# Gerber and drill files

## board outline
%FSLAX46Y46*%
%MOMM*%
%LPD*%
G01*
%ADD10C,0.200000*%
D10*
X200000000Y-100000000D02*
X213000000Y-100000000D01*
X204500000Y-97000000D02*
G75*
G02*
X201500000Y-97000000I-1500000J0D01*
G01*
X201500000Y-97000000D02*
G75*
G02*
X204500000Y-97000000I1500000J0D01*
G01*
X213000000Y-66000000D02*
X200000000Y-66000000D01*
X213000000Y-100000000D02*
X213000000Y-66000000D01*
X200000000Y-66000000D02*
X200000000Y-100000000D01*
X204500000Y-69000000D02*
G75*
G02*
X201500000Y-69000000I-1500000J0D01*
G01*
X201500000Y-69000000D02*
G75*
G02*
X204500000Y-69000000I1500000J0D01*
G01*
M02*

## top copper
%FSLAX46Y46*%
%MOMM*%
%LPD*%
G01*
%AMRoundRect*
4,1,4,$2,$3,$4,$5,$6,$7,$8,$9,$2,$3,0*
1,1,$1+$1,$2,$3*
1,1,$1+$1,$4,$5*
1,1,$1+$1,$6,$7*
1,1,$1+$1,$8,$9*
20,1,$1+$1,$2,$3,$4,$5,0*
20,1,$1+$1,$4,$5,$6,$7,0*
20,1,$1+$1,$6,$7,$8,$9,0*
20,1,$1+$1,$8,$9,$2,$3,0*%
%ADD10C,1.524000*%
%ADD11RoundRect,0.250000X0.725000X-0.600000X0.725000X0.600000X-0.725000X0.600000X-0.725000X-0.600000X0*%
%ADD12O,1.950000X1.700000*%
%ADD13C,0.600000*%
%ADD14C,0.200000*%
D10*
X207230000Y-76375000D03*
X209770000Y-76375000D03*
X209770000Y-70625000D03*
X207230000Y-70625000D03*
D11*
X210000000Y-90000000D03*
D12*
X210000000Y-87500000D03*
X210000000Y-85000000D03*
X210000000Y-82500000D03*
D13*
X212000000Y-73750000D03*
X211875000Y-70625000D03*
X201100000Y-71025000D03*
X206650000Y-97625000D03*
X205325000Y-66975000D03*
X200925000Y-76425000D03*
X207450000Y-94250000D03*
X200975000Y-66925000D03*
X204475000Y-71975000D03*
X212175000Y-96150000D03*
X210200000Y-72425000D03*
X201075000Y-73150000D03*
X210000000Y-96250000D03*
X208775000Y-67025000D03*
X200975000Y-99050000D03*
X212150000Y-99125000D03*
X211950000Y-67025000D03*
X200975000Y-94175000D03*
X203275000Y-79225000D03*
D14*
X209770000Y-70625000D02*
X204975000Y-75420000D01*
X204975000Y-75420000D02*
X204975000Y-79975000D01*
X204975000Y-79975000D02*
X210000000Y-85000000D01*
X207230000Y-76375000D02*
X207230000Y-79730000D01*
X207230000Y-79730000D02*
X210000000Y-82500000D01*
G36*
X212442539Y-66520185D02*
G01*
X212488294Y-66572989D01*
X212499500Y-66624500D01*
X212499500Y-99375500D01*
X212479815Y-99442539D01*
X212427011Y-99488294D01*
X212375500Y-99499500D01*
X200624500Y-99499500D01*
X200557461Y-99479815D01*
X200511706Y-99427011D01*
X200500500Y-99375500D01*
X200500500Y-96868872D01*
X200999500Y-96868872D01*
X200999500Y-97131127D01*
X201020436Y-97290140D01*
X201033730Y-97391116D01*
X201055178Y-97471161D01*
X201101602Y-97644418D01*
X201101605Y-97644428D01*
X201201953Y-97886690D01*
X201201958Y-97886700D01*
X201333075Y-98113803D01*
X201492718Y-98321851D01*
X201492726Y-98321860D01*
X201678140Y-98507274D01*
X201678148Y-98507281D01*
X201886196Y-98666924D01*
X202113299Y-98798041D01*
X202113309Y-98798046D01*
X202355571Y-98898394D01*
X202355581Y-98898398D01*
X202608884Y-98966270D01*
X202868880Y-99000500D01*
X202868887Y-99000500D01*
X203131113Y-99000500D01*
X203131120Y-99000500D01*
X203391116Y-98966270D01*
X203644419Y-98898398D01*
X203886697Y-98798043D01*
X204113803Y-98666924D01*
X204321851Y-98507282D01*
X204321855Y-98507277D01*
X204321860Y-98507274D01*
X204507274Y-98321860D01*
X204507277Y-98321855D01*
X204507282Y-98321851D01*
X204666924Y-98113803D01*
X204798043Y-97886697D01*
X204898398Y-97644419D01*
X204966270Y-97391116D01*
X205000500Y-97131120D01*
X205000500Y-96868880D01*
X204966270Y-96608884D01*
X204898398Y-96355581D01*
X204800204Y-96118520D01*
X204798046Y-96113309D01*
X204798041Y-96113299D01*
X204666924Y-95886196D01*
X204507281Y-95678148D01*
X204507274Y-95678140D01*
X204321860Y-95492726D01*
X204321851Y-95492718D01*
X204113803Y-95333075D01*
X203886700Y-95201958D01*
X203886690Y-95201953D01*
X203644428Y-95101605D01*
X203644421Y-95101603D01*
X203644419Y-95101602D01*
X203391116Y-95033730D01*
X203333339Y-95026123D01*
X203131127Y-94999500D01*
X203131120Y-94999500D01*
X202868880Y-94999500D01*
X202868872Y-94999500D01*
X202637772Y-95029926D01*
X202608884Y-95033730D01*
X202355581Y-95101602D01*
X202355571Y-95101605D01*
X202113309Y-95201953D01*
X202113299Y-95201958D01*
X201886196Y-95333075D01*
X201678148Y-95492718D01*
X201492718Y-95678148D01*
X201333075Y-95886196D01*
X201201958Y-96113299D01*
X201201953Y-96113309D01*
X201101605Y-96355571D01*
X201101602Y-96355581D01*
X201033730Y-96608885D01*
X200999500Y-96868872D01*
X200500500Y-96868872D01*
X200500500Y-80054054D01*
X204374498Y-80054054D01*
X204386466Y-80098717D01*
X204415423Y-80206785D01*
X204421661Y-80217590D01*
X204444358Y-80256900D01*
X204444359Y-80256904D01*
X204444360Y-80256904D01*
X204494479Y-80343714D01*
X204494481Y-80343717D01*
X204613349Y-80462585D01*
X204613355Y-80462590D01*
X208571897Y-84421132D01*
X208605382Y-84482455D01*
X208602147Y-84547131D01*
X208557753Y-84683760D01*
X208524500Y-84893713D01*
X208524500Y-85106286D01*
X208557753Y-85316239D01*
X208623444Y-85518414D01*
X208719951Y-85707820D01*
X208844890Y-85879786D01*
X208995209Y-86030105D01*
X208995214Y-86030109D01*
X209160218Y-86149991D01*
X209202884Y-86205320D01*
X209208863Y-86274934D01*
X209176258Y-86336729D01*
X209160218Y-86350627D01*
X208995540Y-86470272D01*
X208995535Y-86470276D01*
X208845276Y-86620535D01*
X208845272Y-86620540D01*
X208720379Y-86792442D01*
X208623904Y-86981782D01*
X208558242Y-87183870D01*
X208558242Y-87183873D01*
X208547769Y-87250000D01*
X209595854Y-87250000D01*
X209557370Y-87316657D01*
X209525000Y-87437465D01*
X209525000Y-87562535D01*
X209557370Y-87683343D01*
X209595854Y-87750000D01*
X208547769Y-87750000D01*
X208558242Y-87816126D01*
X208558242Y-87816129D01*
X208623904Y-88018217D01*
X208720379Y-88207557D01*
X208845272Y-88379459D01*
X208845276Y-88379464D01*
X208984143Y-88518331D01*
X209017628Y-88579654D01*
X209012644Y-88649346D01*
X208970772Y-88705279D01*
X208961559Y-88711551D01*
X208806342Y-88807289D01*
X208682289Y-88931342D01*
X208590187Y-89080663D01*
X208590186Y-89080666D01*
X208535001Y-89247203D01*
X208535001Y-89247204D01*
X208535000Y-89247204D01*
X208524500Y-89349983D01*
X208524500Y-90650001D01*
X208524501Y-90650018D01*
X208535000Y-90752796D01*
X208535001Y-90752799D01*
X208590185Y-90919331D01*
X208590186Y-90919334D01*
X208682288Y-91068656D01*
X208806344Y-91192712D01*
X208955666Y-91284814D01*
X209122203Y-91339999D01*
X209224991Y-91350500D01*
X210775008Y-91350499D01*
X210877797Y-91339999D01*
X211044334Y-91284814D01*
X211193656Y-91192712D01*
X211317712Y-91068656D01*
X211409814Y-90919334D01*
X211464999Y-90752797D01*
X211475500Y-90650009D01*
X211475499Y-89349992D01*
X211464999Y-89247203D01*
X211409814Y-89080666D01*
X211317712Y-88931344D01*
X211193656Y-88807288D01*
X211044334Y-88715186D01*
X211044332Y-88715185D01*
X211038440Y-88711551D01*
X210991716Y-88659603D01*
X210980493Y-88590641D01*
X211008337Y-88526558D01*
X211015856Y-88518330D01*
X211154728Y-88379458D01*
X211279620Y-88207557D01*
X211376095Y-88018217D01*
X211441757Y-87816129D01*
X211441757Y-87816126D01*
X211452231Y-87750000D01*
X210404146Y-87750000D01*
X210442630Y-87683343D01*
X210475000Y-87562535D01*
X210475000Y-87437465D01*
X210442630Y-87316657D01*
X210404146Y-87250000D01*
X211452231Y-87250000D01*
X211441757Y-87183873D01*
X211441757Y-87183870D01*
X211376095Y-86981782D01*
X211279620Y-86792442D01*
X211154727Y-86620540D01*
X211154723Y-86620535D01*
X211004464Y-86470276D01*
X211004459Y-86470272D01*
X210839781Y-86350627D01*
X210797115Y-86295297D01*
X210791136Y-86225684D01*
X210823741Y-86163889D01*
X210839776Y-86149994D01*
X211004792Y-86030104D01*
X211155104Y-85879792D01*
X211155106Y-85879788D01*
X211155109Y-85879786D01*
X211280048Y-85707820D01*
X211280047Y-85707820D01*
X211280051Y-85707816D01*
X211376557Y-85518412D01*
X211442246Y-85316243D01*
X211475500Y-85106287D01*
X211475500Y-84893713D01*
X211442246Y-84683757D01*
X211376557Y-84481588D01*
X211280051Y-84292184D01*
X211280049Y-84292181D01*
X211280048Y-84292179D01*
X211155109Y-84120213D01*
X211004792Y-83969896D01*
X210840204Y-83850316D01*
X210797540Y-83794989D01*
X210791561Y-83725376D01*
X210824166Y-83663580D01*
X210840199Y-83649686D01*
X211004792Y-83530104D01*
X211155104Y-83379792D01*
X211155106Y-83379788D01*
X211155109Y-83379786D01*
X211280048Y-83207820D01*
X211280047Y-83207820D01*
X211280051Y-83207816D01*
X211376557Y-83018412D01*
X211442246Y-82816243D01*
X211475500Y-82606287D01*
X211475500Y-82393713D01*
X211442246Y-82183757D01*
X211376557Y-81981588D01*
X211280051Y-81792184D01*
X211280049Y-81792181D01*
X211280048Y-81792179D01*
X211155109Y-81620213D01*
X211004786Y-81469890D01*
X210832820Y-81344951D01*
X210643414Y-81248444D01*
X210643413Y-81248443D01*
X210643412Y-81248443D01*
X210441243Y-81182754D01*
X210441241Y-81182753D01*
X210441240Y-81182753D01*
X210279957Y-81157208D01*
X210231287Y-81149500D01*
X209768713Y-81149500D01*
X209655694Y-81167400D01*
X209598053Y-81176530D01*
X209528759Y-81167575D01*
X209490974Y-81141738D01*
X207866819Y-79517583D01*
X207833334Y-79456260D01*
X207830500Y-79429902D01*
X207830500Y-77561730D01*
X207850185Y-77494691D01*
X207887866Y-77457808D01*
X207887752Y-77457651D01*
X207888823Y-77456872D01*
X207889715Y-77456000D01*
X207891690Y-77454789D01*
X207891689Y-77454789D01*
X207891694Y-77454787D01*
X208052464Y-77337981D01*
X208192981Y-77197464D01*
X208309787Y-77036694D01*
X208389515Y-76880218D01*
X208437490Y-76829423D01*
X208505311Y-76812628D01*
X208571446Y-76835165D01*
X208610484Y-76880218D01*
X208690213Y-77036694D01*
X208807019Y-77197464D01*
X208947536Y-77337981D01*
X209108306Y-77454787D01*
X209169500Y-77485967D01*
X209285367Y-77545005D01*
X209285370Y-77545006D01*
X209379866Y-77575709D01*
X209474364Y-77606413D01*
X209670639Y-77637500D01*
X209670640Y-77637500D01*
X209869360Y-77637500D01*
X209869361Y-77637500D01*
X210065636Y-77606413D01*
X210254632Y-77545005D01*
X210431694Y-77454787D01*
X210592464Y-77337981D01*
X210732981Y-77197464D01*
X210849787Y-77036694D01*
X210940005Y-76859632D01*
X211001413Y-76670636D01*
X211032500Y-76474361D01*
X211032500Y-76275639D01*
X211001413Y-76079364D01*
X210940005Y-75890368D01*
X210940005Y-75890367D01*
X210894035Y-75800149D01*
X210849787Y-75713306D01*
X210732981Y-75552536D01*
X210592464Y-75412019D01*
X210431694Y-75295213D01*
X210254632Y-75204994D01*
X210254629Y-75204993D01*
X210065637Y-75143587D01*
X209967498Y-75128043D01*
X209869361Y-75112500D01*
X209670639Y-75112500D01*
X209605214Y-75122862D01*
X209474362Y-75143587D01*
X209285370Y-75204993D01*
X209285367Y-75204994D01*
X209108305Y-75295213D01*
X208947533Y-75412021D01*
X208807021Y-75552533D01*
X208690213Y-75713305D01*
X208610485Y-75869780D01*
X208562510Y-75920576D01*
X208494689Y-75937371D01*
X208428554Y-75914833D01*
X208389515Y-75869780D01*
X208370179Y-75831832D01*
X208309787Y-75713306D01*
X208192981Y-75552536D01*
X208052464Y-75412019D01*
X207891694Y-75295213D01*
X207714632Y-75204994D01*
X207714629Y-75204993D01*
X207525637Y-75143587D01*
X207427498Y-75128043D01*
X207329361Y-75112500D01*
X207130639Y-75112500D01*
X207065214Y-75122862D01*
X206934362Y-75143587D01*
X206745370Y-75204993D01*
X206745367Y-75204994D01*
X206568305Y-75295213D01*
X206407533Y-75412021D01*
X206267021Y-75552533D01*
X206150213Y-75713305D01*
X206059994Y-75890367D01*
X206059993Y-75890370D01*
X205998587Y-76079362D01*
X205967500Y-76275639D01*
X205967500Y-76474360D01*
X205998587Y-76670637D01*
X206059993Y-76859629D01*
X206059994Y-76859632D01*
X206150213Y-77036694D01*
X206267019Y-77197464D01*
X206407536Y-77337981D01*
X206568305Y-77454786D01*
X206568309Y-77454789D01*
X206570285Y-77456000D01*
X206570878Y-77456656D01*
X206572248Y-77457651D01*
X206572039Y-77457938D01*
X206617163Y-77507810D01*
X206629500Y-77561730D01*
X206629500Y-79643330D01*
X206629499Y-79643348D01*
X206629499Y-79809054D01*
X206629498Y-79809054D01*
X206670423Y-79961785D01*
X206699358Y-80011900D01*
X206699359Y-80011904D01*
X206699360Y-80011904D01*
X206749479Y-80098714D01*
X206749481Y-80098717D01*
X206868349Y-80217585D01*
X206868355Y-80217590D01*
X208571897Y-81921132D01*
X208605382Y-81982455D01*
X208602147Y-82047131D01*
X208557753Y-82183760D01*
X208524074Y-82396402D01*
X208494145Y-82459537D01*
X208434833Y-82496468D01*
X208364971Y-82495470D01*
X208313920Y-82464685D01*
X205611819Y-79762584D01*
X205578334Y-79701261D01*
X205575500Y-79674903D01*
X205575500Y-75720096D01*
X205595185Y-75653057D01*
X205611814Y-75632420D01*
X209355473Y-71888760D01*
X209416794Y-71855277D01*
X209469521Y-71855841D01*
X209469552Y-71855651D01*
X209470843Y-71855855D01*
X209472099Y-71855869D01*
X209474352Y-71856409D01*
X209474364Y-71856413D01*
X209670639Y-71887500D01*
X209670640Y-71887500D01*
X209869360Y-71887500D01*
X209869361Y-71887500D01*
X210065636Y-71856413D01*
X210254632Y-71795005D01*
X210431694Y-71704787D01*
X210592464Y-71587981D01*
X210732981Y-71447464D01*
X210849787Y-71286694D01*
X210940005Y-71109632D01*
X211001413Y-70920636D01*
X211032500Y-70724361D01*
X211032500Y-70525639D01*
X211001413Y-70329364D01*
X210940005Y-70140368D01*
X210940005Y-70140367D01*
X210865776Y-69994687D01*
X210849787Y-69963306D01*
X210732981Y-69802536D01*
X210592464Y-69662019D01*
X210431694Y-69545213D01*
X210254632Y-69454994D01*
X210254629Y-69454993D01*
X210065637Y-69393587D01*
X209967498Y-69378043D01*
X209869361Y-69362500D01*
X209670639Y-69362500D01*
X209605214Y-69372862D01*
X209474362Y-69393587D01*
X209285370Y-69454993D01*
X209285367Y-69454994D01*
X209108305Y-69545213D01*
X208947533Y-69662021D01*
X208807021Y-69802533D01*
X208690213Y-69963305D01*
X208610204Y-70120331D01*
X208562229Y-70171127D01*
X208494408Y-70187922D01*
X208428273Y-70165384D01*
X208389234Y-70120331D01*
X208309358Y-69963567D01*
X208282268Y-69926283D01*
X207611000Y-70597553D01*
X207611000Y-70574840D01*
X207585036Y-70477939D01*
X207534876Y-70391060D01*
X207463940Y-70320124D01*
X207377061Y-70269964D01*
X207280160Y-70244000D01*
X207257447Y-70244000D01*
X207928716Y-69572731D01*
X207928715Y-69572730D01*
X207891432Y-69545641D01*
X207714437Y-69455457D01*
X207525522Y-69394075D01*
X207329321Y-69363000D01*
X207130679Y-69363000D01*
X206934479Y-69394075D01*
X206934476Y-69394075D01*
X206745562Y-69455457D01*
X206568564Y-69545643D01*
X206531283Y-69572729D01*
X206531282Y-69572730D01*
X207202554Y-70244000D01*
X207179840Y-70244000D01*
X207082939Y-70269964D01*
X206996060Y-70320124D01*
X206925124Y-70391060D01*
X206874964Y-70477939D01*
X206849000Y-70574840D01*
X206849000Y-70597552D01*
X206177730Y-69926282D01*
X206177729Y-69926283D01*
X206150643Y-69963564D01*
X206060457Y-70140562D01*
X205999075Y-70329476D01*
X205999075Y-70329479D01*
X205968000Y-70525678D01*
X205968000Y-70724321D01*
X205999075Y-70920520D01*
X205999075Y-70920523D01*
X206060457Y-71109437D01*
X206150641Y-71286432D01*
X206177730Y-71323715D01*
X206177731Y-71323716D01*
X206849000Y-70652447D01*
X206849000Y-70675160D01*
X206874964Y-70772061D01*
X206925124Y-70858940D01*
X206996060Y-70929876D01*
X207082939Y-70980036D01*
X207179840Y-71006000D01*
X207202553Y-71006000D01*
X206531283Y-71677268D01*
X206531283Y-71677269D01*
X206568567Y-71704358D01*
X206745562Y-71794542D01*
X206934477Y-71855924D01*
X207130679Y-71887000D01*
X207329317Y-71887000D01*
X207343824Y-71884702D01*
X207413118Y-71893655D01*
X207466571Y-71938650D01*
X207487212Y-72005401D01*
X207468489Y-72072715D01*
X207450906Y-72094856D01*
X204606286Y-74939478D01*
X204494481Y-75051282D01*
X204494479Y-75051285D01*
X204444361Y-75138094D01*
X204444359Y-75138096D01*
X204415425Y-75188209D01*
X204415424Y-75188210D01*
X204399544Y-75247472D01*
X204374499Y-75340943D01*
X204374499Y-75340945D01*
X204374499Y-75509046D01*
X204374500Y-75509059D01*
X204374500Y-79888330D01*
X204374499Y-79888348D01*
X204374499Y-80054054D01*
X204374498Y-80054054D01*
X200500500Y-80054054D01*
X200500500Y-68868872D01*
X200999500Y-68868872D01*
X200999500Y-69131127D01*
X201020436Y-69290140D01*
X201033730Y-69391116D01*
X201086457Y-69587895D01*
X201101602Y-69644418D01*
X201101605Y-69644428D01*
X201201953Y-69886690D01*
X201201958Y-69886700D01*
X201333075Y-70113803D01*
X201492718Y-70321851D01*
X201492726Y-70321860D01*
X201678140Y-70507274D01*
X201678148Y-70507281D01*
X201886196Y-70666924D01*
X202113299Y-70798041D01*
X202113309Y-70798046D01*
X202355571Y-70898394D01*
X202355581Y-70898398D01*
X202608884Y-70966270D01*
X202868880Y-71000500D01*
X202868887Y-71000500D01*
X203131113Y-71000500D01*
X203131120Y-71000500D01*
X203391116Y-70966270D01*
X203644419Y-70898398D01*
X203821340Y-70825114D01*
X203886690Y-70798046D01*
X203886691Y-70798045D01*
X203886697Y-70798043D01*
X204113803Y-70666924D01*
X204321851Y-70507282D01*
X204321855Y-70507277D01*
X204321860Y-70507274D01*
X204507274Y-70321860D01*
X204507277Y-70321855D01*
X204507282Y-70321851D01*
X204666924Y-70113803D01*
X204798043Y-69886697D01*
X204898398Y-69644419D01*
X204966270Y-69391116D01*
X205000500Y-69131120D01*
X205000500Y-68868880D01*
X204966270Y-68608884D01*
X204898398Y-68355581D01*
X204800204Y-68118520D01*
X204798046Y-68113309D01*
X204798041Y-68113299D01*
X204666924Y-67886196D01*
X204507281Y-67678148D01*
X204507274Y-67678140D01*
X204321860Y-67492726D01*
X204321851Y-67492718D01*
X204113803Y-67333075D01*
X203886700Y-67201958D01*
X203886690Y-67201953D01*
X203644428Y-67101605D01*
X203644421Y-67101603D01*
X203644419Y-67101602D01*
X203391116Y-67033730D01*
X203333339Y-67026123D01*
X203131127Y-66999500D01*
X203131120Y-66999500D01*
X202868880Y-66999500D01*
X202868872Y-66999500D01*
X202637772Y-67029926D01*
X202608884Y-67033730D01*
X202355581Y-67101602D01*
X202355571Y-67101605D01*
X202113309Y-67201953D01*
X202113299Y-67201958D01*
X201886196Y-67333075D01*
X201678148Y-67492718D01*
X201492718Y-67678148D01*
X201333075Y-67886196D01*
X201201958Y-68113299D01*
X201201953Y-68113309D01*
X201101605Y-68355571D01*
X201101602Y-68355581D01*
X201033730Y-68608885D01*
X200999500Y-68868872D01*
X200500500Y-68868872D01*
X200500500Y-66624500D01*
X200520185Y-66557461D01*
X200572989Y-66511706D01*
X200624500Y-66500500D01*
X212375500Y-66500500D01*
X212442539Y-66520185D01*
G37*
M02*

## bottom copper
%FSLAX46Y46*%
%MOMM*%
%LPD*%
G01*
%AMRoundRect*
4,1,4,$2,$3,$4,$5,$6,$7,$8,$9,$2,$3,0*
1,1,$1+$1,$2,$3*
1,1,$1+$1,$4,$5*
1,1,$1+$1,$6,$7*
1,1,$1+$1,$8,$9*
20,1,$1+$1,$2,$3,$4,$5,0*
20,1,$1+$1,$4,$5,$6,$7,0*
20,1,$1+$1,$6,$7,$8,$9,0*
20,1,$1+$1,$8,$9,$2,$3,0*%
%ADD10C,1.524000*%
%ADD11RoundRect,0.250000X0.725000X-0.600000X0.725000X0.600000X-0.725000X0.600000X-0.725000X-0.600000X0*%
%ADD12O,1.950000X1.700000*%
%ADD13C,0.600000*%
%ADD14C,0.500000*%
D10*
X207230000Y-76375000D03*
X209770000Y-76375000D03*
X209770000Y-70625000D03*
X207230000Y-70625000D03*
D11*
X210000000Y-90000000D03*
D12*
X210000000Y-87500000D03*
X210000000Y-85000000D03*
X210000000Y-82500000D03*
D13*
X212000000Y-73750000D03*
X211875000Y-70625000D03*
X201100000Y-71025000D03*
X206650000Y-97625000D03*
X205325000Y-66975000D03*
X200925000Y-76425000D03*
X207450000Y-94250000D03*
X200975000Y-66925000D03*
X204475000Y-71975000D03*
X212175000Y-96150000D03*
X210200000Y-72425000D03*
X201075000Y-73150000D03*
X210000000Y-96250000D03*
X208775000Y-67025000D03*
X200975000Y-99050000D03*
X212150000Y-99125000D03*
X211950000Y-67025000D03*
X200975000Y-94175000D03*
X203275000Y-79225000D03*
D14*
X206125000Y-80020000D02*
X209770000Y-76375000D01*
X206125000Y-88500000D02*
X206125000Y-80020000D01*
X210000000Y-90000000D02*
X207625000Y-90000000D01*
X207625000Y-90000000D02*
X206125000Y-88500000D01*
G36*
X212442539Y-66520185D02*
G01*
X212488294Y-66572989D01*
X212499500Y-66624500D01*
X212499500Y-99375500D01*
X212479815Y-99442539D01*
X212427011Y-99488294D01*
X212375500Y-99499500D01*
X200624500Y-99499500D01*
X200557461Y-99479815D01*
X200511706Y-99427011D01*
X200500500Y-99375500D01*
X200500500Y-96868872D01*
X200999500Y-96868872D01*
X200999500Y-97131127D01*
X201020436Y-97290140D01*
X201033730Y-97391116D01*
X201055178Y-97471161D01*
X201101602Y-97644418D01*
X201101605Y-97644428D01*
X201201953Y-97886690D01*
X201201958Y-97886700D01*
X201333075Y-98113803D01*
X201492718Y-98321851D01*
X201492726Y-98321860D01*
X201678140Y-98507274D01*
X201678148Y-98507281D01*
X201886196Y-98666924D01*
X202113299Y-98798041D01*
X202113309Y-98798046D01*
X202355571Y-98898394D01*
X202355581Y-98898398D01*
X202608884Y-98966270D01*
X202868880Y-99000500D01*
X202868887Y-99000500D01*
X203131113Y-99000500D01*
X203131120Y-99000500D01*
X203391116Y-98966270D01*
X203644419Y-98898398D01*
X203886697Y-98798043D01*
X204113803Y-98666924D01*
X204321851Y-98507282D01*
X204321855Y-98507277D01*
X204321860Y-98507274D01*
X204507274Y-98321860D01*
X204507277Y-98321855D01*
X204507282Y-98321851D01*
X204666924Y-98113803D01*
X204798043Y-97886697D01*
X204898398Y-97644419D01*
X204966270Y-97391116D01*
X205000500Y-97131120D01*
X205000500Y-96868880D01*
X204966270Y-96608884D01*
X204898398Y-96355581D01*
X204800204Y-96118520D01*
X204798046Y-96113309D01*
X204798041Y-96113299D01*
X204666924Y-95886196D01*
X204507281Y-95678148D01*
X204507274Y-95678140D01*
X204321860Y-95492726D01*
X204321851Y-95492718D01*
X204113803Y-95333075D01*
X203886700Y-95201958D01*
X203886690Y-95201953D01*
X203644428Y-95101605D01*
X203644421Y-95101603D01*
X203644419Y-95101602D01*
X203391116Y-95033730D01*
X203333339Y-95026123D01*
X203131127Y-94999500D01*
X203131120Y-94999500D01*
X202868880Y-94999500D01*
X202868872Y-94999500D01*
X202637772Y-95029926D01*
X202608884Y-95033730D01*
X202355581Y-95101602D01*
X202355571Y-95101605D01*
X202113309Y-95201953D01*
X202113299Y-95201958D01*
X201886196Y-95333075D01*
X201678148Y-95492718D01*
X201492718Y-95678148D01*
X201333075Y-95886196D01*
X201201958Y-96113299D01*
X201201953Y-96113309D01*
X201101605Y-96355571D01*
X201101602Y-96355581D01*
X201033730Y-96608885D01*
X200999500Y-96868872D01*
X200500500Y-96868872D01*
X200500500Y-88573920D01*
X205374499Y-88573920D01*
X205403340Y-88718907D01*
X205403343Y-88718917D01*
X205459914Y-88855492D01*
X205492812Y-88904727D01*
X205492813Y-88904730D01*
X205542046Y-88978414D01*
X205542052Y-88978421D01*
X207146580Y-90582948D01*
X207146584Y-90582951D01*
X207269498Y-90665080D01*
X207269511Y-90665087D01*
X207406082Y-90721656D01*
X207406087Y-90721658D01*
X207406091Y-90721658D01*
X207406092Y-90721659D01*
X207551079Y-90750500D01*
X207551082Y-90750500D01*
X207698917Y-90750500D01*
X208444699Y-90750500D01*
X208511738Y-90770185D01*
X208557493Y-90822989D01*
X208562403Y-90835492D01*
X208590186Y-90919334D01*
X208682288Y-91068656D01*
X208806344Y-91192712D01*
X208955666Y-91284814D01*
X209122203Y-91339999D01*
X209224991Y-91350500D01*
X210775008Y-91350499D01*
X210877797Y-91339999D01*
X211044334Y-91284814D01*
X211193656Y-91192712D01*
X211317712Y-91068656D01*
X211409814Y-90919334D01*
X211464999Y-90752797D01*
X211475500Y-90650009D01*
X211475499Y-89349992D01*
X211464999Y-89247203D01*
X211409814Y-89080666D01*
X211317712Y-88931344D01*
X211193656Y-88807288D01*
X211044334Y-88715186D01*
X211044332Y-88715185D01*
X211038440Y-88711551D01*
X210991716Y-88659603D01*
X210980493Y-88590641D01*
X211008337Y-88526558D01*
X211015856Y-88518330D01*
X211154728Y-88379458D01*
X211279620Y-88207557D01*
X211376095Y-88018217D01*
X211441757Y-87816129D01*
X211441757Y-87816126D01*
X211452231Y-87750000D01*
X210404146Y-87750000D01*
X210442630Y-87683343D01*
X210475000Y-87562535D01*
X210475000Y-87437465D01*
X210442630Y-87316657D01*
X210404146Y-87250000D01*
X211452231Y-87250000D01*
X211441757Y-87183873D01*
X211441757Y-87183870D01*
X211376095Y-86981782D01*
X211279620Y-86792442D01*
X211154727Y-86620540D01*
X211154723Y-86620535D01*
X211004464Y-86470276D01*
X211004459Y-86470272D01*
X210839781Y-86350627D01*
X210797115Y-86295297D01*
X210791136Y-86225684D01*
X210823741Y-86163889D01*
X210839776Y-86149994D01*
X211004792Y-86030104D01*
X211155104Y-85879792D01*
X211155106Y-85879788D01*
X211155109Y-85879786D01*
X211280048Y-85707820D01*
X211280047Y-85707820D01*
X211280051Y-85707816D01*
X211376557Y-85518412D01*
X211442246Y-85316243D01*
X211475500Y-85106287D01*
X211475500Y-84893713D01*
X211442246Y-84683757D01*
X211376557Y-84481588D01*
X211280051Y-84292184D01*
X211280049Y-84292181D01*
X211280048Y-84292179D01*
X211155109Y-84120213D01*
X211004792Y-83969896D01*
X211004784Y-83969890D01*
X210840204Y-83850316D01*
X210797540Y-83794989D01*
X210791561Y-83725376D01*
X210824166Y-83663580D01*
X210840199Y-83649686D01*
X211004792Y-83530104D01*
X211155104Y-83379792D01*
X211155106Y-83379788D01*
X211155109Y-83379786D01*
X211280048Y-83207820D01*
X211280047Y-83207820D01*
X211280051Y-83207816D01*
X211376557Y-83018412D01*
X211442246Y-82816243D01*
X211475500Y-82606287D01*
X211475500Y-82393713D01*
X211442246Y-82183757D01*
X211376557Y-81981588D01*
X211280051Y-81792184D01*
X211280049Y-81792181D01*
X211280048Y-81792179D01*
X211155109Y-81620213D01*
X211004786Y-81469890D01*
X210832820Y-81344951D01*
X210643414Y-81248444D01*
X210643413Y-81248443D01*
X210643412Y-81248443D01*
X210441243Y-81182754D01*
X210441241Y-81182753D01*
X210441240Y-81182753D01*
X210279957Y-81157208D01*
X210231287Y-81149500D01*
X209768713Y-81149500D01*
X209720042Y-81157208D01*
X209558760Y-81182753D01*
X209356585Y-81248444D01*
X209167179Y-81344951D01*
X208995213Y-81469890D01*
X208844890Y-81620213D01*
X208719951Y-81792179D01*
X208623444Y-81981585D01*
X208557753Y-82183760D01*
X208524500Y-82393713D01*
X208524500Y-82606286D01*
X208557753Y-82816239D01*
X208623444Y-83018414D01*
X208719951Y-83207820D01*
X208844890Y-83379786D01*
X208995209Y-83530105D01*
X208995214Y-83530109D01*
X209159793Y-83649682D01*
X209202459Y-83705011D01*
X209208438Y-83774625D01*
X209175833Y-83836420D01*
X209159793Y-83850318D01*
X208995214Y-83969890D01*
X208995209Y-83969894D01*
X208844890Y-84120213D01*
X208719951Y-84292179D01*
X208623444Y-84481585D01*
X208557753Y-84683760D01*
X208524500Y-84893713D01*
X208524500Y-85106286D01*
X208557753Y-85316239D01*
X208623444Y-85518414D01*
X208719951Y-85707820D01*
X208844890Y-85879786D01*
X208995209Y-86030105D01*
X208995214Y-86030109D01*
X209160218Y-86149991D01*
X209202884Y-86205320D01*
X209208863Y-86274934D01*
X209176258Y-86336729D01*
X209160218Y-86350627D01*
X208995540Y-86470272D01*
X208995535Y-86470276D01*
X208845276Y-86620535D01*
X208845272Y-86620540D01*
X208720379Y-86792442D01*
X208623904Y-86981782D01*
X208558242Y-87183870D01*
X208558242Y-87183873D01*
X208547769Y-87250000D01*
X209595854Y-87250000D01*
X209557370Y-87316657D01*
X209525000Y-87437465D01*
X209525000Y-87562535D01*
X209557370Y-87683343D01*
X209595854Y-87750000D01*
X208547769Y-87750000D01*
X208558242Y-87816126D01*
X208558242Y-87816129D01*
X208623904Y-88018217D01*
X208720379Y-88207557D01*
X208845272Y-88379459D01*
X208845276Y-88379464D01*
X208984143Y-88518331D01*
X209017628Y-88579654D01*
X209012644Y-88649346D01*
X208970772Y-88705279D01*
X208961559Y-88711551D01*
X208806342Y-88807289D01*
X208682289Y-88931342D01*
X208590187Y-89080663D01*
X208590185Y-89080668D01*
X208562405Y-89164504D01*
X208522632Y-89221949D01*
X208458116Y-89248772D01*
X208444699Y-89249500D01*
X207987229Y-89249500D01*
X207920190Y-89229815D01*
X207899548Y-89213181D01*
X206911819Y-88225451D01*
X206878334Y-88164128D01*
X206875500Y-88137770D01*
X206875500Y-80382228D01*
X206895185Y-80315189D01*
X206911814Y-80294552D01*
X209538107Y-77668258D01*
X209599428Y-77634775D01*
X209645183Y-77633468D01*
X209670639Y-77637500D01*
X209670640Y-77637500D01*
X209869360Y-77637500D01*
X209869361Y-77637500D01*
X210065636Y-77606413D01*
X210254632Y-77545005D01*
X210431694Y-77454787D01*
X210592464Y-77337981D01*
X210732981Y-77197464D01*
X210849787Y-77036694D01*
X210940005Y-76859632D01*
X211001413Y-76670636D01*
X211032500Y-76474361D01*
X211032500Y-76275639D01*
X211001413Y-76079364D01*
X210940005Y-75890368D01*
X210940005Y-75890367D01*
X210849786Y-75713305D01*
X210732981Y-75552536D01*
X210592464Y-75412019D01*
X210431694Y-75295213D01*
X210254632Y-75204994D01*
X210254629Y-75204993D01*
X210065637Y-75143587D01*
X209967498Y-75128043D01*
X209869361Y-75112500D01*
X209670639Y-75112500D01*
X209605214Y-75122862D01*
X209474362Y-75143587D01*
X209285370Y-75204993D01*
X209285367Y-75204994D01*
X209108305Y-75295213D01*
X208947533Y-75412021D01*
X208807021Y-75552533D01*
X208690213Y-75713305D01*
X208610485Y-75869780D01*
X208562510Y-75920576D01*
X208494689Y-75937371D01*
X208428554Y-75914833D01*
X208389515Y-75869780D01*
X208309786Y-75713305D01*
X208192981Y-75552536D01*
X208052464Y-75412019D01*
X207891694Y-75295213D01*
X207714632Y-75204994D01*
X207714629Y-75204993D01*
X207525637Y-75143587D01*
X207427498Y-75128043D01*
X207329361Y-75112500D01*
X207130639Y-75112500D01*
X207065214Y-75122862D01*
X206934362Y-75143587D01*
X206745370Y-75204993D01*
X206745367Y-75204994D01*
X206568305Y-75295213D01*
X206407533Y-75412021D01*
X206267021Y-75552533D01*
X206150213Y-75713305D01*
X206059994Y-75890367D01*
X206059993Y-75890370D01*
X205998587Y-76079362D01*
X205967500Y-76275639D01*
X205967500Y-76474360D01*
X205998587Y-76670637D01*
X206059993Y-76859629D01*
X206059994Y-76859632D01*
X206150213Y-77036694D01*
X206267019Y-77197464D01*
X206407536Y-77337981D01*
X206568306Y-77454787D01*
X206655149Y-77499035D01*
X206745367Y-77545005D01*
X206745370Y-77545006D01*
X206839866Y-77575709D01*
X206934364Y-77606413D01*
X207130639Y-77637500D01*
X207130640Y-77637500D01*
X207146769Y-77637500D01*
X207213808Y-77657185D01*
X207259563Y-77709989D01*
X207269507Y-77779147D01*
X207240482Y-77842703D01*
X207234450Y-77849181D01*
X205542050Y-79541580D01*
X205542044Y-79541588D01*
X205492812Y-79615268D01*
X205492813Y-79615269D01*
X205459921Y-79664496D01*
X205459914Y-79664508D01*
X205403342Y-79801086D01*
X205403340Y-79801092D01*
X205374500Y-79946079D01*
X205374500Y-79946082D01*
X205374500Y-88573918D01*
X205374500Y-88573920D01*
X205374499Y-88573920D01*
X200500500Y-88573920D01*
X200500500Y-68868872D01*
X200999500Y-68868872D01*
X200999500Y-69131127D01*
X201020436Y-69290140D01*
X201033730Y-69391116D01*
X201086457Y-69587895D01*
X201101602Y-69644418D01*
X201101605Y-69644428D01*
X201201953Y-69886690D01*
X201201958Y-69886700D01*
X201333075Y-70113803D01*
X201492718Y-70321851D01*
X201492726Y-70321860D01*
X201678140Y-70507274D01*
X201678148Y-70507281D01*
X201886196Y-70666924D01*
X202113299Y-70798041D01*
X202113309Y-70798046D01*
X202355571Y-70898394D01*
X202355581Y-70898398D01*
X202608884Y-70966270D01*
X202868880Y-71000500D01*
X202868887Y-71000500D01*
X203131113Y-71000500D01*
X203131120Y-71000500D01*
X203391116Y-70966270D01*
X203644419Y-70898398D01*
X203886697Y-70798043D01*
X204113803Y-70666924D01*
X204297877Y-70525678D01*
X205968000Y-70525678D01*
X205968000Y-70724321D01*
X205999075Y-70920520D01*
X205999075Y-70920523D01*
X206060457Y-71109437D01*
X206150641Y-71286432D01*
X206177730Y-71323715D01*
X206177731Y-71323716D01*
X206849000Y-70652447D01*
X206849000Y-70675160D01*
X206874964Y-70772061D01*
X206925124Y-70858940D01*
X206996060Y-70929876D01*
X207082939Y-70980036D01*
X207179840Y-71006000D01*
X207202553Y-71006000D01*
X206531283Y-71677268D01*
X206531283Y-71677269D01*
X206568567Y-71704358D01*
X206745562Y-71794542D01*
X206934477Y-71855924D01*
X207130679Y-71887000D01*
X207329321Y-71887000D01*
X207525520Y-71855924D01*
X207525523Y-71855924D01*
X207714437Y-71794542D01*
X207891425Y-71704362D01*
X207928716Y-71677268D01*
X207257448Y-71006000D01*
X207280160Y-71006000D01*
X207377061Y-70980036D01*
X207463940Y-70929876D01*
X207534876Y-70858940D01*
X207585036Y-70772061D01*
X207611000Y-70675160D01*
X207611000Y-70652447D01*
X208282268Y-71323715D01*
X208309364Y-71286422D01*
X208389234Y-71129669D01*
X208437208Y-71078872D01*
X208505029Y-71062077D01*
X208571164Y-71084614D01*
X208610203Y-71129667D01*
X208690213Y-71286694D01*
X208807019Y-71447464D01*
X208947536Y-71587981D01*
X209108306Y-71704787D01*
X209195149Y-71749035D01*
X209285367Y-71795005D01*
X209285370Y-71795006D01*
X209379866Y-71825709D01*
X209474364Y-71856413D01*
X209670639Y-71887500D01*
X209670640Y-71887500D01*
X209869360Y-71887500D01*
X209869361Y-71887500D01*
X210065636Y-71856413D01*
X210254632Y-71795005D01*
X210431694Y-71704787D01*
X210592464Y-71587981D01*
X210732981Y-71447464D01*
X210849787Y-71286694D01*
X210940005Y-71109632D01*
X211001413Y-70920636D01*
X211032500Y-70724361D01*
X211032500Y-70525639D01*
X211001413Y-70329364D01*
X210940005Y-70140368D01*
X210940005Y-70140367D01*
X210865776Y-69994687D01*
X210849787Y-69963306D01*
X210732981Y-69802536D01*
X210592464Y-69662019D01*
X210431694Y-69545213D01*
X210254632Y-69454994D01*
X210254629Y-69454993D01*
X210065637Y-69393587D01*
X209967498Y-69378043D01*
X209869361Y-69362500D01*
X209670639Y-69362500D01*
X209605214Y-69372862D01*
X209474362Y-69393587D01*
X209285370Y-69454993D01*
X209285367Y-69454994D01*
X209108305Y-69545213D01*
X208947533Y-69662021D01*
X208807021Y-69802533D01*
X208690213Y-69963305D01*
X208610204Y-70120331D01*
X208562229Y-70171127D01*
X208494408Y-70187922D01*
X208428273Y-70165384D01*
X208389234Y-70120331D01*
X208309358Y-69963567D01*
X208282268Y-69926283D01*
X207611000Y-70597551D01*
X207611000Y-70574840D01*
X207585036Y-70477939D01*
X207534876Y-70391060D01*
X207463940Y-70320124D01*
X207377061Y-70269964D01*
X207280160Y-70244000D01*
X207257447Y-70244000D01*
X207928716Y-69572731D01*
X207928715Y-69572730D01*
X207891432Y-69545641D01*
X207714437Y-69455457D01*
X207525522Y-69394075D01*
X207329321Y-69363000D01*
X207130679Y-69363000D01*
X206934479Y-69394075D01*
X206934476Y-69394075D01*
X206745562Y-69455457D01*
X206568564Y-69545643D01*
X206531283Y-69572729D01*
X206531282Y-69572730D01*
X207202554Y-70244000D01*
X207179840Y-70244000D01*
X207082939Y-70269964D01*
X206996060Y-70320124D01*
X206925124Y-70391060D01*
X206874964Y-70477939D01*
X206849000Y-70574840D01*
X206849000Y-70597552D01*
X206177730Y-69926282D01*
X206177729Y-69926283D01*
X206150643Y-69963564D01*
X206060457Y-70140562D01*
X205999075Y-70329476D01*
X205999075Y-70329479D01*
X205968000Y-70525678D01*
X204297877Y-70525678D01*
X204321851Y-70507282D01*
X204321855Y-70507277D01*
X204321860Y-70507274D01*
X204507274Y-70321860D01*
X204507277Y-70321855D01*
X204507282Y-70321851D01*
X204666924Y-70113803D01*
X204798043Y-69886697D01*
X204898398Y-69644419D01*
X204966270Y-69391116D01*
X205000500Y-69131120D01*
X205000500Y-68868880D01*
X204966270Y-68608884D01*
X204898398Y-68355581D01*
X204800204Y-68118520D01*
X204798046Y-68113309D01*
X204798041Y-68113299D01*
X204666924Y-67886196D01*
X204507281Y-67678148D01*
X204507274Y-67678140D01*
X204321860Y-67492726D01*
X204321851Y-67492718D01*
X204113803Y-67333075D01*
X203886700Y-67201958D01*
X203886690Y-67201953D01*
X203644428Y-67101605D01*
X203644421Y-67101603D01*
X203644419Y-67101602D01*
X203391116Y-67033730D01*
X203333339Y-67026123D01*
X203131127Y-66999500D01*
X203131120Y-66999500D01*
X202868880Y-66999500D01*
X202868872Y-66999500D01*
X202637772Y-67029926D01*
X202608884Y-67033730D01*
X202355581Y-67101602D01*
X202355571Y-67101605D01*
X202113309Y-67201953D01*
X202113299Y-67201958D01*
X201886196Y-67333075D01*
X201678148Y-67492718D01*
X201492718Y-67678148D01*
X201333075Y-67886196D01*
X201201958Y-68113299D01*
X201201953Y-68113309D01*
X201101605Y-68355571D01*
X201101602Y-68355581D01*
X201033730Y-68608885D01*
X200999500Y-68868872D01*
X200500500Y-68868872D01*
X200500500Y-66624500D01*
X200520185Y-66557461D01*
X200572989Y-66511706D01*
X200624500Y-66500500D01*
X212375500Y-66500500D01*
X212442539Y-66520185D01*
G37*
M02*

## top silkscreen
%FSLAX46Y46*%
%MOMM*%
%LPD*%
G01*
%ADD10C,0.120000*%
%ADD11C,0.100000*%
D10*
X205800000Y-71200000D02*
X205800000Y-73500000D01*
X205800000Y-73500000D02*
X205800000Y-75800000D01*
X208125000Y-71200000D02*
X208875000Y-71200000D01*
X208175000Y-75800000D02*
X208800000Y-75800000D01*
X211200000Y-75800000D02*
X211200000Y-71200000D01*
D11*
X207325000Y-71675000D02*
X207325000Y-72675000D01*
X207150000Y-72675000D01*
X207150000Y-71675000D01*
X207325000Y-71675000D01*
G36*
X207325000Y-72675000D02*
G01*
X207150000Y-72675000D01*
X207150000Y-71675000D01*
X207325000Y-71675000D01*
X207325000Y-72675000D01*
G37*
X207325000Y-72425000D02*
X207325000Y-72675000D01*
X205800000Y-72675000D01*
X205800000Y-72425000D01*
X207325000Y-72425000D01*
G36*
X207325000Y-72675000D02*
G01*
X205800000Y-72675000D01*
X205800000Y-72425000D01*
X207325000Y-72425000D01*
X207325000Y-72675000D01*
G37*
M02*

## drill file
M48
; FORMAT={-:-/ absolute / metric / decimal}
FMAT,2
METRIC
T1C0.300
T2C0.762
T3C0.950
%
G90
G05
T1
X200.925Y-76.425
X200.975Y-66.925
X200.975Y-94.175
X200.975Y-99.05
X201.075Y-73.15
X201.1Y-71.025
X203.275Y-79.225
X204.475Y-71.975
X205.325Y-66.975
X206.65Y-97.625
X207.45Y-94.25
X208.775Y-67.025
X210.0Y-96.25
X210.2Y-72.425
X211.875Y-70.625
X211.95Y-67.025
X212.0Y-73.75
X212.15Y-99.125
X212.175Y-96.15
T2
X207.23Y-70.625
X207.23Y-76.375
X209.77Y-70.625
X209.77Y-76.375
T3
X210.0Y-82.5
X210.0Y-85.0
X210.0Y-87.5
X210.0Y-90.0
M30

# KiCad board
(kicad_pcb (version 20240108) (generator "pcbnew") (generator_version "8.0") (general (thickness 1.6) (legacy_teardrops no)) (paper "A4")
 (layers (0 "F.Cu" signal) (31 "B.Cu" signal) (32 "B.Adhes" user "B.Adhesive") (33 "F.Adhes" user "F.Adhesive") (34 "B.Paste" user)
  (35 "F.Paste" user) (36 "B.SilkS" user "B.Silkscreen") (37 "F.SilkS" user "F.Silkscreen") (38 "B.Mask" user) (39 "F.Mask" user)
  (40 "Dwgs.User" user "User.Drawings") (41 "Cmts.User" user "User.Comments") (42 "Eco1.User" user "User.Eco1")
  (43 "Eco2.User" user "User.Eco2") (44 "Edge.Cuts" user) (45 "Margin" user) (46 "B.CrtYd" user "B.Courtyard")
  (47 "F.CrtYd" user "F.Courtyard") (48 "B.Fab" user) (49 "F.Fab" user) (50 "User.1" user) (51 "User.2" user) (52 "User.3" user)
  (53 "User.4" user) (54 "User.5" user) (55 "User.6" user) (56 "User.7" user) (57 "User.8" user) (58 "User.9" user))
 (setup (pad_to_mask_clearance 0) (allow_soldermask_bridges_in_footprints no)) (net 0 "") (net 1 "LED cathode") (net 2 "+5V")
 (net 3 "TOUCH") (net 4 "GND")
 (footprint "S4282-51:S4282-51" (layer "F.Cu") (at 208.5 73.5 90)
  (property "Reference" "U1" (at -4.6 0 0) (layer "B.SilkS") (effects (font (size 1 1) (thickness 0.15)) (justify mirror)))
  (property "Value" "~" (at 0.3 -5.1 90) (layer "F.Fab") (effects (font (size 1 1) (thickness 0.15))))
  (fp_line (start 2.3 -2.7) (end 0 -2.7) (stroke (width 0.12) (type solid)) (layer "F.SilkS"))
  (fp_line (start 0 -2.7) (end -2.3 -2.7) (stroke (width 0.12) (type solid)) (layer "F.SilkS"))
  (fp_line (start 2.3 -0.375) (end 2.3 0.375) (stroke (width 0.12) (type solid)) (layer "F.SilkS"))
  (fp_line (start -2.3 -0.325) (end -2.3 0.3) (stroke (width 0.12) (type solid)) (layer "F.SilkS"))
  (fp_line (start -2.3 2.7) (end 2.3 2.7) (stroke (width 0.12) (type solid)) (layer "F.SilkS"))
  (fp_poly
   (pts (xy 1.825 -1.175) (xy 0.825 -1.175) (xy 0.825 -1.35) (xy 1.825 -1.35)) (stroke (width 0.1) (type solid)) (fill solid)
   (layer "F.SilkS"))
  (fp_poly
   (pts (xy 1.075 -1.175) (xy 0.825 -1.175) (xy 0.825 -2.7) (xy 1.075 -2.7)) (stroke (width 0.1) (type solid)) (fill solid)
   (layer "F.SilkS"))
  (pad "1" thru_hole circle (at -2.875 -1.27 90) (size 1.524 1.524) (drill 0.762) (layers "*.Cu" "*.Mask") (remove_unused_layers no)
   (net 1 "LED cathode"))
  (pad "2" thru_hole circle (at -2.875 1.27 90) (size 1.524 1.524) (drill 0.762) (layers "*.Cu" "*.Mask") (remove_unused_layers no)
   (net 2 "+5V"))
  (pad "3" thru_hole circle (at 2.875 1.27 90) (size 1.524 1.524) (drill 0.762) (layers "*.Cu" "*.Mask") (remove_unused_layers no)
   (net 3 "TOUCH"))
  (pad "4" thru_hole circle (at 2.875 -1.27 90) (size 1.524 1.524) (drill 0.762) (layers "*.Cu" "*.Mask") (remove_unused_layers no)
   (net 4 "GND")))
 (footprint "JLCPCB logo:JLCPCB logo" (layer "B.Cu") (at 206.5 94 180)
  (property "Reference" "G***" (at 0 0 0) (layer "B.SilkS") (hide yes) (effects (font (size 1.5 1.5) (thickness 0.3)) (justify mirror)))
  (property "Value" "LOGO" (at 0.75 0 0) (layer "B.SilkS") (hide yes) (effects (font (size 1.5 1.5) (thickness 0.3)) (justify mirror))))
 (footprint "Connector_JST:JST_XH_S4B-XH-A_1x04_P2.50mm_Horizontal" (layer "B.Cu") (at 210 90 90)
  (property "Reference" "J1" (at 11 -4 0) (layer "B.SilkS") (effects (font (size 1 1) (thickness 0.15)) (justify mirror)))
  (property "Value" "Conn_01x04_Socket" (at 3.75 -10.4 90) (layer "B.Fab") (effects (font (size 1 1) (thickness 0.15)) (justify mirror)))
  (pad "1" thru_hole roundrect (at 0 0 90) (size 1.7 1.95) (drill 0.95) (layers "*.Cu" "*.Mask") (remove_unused_layers no)
   (roundrect_rratio 0.147059) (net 2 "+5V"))
  (pad "2" thru_hole oval (at 2.5 0 90) (size 1.7 1.95) (drill 0.95) (layers "*.Cu" "*.Mask") (remove_unused_layers no) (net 4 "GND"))
  (pad "3" thru_hole oval (at 5 0 90) (size 1.7 1.95) (drill 0.95) (layers "*.Cu" "*.Mask") (remove_unused_layers no) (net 3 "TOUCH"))
  (pad "4" thru_hole oval (at 7.5 0 90) (size 1.7 1.95) (drill 0.95) (layers "*.Cu" "*.Mask") (remove_unused_layers no)
   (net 1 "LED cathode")))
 (gr_line (start 200 100) (end 213 100) (stroke (width 0.2) (type default)) (layer "Edge.Cuts"))
 (gr_circle (center 203 97) (end 204.5 97) (stroke (width 0.2) (type default)) (fill none) (layer "Edge.Cuts"))
 (gr_line (start 213 66) (end 200 66) (stroke (width 0.2) (type default)) (layer "Edge.Cuts"))
 (gr_line (start 213 100) (end 213 66) (stroke (width 0.2) (type default)) (layer "Edge.Cuts"))
 (gr_line (start 200 66) (end 200 100) (stroke (width 0.2) (type default)) (layer "Edge.Cuts"))
 (gr_circle (center 203 69) (end 204.5 69) (stroke (width 0.2) (type default)) (fill none) (layer "Edge.Cuts"))
 (segment (start 206.125 80.02) (end 209.77 76.375) (width 0.5) (layer "B.Cu") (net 2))
 (segment (start 206.125 88.5) (end 206.125 80.02) (width 0.5) (layer "B.Cu") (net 2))
 (segment (start 210 90) (end 207.625 90) (width 0.5) (layer "B.Cu") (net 2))
 (segment (start 207.625 90) (end 206.125 88.5) (width 0.5) (layer "B.Cu") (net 2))
 (via (at 212 73.75) (size 0.6) (drill 0.3) (layers "F.Cu" "B.Cu") (free yes) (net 4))
 (via (at 211.875 70.625) (size 0.6) (drill 0.3) (layers "F.Cu" "B.Cu") (free yes) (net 4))
 (via (at 201.1 71.025) (size 0.6) (drill 0.3) (layers "F.Cu" "B.Cu") (free yes) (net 4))
 (via (at 206.65 97.625) (size 0.6) (drill 0.3) (layers "F.Cu" "B.Cu") (free yes) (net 4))
 (via (at 205.325 66.975) (size 0.6) (drill 0.3) (layers "F.Cu" "B.Cu") (free yes) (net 4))
 (via (at 200.925 76.425) (size 0.6) (drill 0.3) (layers "F.Cu" "B.Cu") (free yes) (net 4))
 (via (at 207.45 94.25) (size 0.6) (drill 0.3) (layers "F.Cu" "B.Cu") (free yes) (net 4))
 (via (at 200.975 66.925) (size 0.6) (drill 0.3) (layers "F.Cu" "B.Cu") (free yes) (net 4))
 (via (at 204.475 71.975) (size 0.6) (drill 0.3) (layers "F.Cu" "B.Cu") (free yes) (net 4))
 (via (at 212.175 96.15) (size 0.6) (drill 0.3) (layers "F.Cu" "B.Cu") (free yes) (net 4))
 (via (at 210.2 72.425) (size 0.6) (drill 0.3) (layers "F.Cu" "B.Cu") (free yes) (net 4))
 (via (at 201.075 73.15) (size 0.6) (drill 0.3) (layers "F.Cu" "B.Cu") (free yes) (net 4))
 (via (at 210 96.25) (size 0.6) (drill 0.3) (layers "F.Cu" "B.Cu") (free yes) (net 4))
 (via (at 208.775 67.025) (size 0.6) (drill 0.3) (layers "F.Cu" "B.Cu") (free yes) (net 4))
 (via (at 200.975 99.05) (size 0.6) (drill 0.3) (layers "F.Cu" "B.Cu") (free yes) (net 4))
 (via (at 212.15 99.125) (size 0.6) (drill 0.3) (layers "F.Cu" "B.Cu") (free yes) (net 4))
 (via (at 211.95 67.025) (size 0.6) (drill 0.3) (layers "F.Cu" "B.Cu") (free yes) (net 4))
 (via (at 200.975 94.175) (size 0.6) (drill 0.3) (layers "F.Cu" "B.Cu") (free yes) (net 4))
 (via (at 203.275 79.225) (size 0.6) (drill 0.3) (layers "F.Cu" "B.Cu") (free yes) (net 4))
 (segment (start 209.77 70.625) (end 204.975 75.42) (width 0.2) (layer "F.Cu") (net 3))
 (segment (start 204.975 75.42) (end 204.975 79.975) (width 0.2) (layer "F.Cu") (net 3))
 (segment (start 204.975 79.975) (end 210 85) (width 0.2) (layer "F.Cu") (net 3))
 (segment (start 207.23 76.375) (end 207.23 79.73) (width 0.2) (layer "F.Cu") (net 1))
 (segment (start 207.23 79.73) (end 210 82.5) (width 0.2) (layer "F.Cu") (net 1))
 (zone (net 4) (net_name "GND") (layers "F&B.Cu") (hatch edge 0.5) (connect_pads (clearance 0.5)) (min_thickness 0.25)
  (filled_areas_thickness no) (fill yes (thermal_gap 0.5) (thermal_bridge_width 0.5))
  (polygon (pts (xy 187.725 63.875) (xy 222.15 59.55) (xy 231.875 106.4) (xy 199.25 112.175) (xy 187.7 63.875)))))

